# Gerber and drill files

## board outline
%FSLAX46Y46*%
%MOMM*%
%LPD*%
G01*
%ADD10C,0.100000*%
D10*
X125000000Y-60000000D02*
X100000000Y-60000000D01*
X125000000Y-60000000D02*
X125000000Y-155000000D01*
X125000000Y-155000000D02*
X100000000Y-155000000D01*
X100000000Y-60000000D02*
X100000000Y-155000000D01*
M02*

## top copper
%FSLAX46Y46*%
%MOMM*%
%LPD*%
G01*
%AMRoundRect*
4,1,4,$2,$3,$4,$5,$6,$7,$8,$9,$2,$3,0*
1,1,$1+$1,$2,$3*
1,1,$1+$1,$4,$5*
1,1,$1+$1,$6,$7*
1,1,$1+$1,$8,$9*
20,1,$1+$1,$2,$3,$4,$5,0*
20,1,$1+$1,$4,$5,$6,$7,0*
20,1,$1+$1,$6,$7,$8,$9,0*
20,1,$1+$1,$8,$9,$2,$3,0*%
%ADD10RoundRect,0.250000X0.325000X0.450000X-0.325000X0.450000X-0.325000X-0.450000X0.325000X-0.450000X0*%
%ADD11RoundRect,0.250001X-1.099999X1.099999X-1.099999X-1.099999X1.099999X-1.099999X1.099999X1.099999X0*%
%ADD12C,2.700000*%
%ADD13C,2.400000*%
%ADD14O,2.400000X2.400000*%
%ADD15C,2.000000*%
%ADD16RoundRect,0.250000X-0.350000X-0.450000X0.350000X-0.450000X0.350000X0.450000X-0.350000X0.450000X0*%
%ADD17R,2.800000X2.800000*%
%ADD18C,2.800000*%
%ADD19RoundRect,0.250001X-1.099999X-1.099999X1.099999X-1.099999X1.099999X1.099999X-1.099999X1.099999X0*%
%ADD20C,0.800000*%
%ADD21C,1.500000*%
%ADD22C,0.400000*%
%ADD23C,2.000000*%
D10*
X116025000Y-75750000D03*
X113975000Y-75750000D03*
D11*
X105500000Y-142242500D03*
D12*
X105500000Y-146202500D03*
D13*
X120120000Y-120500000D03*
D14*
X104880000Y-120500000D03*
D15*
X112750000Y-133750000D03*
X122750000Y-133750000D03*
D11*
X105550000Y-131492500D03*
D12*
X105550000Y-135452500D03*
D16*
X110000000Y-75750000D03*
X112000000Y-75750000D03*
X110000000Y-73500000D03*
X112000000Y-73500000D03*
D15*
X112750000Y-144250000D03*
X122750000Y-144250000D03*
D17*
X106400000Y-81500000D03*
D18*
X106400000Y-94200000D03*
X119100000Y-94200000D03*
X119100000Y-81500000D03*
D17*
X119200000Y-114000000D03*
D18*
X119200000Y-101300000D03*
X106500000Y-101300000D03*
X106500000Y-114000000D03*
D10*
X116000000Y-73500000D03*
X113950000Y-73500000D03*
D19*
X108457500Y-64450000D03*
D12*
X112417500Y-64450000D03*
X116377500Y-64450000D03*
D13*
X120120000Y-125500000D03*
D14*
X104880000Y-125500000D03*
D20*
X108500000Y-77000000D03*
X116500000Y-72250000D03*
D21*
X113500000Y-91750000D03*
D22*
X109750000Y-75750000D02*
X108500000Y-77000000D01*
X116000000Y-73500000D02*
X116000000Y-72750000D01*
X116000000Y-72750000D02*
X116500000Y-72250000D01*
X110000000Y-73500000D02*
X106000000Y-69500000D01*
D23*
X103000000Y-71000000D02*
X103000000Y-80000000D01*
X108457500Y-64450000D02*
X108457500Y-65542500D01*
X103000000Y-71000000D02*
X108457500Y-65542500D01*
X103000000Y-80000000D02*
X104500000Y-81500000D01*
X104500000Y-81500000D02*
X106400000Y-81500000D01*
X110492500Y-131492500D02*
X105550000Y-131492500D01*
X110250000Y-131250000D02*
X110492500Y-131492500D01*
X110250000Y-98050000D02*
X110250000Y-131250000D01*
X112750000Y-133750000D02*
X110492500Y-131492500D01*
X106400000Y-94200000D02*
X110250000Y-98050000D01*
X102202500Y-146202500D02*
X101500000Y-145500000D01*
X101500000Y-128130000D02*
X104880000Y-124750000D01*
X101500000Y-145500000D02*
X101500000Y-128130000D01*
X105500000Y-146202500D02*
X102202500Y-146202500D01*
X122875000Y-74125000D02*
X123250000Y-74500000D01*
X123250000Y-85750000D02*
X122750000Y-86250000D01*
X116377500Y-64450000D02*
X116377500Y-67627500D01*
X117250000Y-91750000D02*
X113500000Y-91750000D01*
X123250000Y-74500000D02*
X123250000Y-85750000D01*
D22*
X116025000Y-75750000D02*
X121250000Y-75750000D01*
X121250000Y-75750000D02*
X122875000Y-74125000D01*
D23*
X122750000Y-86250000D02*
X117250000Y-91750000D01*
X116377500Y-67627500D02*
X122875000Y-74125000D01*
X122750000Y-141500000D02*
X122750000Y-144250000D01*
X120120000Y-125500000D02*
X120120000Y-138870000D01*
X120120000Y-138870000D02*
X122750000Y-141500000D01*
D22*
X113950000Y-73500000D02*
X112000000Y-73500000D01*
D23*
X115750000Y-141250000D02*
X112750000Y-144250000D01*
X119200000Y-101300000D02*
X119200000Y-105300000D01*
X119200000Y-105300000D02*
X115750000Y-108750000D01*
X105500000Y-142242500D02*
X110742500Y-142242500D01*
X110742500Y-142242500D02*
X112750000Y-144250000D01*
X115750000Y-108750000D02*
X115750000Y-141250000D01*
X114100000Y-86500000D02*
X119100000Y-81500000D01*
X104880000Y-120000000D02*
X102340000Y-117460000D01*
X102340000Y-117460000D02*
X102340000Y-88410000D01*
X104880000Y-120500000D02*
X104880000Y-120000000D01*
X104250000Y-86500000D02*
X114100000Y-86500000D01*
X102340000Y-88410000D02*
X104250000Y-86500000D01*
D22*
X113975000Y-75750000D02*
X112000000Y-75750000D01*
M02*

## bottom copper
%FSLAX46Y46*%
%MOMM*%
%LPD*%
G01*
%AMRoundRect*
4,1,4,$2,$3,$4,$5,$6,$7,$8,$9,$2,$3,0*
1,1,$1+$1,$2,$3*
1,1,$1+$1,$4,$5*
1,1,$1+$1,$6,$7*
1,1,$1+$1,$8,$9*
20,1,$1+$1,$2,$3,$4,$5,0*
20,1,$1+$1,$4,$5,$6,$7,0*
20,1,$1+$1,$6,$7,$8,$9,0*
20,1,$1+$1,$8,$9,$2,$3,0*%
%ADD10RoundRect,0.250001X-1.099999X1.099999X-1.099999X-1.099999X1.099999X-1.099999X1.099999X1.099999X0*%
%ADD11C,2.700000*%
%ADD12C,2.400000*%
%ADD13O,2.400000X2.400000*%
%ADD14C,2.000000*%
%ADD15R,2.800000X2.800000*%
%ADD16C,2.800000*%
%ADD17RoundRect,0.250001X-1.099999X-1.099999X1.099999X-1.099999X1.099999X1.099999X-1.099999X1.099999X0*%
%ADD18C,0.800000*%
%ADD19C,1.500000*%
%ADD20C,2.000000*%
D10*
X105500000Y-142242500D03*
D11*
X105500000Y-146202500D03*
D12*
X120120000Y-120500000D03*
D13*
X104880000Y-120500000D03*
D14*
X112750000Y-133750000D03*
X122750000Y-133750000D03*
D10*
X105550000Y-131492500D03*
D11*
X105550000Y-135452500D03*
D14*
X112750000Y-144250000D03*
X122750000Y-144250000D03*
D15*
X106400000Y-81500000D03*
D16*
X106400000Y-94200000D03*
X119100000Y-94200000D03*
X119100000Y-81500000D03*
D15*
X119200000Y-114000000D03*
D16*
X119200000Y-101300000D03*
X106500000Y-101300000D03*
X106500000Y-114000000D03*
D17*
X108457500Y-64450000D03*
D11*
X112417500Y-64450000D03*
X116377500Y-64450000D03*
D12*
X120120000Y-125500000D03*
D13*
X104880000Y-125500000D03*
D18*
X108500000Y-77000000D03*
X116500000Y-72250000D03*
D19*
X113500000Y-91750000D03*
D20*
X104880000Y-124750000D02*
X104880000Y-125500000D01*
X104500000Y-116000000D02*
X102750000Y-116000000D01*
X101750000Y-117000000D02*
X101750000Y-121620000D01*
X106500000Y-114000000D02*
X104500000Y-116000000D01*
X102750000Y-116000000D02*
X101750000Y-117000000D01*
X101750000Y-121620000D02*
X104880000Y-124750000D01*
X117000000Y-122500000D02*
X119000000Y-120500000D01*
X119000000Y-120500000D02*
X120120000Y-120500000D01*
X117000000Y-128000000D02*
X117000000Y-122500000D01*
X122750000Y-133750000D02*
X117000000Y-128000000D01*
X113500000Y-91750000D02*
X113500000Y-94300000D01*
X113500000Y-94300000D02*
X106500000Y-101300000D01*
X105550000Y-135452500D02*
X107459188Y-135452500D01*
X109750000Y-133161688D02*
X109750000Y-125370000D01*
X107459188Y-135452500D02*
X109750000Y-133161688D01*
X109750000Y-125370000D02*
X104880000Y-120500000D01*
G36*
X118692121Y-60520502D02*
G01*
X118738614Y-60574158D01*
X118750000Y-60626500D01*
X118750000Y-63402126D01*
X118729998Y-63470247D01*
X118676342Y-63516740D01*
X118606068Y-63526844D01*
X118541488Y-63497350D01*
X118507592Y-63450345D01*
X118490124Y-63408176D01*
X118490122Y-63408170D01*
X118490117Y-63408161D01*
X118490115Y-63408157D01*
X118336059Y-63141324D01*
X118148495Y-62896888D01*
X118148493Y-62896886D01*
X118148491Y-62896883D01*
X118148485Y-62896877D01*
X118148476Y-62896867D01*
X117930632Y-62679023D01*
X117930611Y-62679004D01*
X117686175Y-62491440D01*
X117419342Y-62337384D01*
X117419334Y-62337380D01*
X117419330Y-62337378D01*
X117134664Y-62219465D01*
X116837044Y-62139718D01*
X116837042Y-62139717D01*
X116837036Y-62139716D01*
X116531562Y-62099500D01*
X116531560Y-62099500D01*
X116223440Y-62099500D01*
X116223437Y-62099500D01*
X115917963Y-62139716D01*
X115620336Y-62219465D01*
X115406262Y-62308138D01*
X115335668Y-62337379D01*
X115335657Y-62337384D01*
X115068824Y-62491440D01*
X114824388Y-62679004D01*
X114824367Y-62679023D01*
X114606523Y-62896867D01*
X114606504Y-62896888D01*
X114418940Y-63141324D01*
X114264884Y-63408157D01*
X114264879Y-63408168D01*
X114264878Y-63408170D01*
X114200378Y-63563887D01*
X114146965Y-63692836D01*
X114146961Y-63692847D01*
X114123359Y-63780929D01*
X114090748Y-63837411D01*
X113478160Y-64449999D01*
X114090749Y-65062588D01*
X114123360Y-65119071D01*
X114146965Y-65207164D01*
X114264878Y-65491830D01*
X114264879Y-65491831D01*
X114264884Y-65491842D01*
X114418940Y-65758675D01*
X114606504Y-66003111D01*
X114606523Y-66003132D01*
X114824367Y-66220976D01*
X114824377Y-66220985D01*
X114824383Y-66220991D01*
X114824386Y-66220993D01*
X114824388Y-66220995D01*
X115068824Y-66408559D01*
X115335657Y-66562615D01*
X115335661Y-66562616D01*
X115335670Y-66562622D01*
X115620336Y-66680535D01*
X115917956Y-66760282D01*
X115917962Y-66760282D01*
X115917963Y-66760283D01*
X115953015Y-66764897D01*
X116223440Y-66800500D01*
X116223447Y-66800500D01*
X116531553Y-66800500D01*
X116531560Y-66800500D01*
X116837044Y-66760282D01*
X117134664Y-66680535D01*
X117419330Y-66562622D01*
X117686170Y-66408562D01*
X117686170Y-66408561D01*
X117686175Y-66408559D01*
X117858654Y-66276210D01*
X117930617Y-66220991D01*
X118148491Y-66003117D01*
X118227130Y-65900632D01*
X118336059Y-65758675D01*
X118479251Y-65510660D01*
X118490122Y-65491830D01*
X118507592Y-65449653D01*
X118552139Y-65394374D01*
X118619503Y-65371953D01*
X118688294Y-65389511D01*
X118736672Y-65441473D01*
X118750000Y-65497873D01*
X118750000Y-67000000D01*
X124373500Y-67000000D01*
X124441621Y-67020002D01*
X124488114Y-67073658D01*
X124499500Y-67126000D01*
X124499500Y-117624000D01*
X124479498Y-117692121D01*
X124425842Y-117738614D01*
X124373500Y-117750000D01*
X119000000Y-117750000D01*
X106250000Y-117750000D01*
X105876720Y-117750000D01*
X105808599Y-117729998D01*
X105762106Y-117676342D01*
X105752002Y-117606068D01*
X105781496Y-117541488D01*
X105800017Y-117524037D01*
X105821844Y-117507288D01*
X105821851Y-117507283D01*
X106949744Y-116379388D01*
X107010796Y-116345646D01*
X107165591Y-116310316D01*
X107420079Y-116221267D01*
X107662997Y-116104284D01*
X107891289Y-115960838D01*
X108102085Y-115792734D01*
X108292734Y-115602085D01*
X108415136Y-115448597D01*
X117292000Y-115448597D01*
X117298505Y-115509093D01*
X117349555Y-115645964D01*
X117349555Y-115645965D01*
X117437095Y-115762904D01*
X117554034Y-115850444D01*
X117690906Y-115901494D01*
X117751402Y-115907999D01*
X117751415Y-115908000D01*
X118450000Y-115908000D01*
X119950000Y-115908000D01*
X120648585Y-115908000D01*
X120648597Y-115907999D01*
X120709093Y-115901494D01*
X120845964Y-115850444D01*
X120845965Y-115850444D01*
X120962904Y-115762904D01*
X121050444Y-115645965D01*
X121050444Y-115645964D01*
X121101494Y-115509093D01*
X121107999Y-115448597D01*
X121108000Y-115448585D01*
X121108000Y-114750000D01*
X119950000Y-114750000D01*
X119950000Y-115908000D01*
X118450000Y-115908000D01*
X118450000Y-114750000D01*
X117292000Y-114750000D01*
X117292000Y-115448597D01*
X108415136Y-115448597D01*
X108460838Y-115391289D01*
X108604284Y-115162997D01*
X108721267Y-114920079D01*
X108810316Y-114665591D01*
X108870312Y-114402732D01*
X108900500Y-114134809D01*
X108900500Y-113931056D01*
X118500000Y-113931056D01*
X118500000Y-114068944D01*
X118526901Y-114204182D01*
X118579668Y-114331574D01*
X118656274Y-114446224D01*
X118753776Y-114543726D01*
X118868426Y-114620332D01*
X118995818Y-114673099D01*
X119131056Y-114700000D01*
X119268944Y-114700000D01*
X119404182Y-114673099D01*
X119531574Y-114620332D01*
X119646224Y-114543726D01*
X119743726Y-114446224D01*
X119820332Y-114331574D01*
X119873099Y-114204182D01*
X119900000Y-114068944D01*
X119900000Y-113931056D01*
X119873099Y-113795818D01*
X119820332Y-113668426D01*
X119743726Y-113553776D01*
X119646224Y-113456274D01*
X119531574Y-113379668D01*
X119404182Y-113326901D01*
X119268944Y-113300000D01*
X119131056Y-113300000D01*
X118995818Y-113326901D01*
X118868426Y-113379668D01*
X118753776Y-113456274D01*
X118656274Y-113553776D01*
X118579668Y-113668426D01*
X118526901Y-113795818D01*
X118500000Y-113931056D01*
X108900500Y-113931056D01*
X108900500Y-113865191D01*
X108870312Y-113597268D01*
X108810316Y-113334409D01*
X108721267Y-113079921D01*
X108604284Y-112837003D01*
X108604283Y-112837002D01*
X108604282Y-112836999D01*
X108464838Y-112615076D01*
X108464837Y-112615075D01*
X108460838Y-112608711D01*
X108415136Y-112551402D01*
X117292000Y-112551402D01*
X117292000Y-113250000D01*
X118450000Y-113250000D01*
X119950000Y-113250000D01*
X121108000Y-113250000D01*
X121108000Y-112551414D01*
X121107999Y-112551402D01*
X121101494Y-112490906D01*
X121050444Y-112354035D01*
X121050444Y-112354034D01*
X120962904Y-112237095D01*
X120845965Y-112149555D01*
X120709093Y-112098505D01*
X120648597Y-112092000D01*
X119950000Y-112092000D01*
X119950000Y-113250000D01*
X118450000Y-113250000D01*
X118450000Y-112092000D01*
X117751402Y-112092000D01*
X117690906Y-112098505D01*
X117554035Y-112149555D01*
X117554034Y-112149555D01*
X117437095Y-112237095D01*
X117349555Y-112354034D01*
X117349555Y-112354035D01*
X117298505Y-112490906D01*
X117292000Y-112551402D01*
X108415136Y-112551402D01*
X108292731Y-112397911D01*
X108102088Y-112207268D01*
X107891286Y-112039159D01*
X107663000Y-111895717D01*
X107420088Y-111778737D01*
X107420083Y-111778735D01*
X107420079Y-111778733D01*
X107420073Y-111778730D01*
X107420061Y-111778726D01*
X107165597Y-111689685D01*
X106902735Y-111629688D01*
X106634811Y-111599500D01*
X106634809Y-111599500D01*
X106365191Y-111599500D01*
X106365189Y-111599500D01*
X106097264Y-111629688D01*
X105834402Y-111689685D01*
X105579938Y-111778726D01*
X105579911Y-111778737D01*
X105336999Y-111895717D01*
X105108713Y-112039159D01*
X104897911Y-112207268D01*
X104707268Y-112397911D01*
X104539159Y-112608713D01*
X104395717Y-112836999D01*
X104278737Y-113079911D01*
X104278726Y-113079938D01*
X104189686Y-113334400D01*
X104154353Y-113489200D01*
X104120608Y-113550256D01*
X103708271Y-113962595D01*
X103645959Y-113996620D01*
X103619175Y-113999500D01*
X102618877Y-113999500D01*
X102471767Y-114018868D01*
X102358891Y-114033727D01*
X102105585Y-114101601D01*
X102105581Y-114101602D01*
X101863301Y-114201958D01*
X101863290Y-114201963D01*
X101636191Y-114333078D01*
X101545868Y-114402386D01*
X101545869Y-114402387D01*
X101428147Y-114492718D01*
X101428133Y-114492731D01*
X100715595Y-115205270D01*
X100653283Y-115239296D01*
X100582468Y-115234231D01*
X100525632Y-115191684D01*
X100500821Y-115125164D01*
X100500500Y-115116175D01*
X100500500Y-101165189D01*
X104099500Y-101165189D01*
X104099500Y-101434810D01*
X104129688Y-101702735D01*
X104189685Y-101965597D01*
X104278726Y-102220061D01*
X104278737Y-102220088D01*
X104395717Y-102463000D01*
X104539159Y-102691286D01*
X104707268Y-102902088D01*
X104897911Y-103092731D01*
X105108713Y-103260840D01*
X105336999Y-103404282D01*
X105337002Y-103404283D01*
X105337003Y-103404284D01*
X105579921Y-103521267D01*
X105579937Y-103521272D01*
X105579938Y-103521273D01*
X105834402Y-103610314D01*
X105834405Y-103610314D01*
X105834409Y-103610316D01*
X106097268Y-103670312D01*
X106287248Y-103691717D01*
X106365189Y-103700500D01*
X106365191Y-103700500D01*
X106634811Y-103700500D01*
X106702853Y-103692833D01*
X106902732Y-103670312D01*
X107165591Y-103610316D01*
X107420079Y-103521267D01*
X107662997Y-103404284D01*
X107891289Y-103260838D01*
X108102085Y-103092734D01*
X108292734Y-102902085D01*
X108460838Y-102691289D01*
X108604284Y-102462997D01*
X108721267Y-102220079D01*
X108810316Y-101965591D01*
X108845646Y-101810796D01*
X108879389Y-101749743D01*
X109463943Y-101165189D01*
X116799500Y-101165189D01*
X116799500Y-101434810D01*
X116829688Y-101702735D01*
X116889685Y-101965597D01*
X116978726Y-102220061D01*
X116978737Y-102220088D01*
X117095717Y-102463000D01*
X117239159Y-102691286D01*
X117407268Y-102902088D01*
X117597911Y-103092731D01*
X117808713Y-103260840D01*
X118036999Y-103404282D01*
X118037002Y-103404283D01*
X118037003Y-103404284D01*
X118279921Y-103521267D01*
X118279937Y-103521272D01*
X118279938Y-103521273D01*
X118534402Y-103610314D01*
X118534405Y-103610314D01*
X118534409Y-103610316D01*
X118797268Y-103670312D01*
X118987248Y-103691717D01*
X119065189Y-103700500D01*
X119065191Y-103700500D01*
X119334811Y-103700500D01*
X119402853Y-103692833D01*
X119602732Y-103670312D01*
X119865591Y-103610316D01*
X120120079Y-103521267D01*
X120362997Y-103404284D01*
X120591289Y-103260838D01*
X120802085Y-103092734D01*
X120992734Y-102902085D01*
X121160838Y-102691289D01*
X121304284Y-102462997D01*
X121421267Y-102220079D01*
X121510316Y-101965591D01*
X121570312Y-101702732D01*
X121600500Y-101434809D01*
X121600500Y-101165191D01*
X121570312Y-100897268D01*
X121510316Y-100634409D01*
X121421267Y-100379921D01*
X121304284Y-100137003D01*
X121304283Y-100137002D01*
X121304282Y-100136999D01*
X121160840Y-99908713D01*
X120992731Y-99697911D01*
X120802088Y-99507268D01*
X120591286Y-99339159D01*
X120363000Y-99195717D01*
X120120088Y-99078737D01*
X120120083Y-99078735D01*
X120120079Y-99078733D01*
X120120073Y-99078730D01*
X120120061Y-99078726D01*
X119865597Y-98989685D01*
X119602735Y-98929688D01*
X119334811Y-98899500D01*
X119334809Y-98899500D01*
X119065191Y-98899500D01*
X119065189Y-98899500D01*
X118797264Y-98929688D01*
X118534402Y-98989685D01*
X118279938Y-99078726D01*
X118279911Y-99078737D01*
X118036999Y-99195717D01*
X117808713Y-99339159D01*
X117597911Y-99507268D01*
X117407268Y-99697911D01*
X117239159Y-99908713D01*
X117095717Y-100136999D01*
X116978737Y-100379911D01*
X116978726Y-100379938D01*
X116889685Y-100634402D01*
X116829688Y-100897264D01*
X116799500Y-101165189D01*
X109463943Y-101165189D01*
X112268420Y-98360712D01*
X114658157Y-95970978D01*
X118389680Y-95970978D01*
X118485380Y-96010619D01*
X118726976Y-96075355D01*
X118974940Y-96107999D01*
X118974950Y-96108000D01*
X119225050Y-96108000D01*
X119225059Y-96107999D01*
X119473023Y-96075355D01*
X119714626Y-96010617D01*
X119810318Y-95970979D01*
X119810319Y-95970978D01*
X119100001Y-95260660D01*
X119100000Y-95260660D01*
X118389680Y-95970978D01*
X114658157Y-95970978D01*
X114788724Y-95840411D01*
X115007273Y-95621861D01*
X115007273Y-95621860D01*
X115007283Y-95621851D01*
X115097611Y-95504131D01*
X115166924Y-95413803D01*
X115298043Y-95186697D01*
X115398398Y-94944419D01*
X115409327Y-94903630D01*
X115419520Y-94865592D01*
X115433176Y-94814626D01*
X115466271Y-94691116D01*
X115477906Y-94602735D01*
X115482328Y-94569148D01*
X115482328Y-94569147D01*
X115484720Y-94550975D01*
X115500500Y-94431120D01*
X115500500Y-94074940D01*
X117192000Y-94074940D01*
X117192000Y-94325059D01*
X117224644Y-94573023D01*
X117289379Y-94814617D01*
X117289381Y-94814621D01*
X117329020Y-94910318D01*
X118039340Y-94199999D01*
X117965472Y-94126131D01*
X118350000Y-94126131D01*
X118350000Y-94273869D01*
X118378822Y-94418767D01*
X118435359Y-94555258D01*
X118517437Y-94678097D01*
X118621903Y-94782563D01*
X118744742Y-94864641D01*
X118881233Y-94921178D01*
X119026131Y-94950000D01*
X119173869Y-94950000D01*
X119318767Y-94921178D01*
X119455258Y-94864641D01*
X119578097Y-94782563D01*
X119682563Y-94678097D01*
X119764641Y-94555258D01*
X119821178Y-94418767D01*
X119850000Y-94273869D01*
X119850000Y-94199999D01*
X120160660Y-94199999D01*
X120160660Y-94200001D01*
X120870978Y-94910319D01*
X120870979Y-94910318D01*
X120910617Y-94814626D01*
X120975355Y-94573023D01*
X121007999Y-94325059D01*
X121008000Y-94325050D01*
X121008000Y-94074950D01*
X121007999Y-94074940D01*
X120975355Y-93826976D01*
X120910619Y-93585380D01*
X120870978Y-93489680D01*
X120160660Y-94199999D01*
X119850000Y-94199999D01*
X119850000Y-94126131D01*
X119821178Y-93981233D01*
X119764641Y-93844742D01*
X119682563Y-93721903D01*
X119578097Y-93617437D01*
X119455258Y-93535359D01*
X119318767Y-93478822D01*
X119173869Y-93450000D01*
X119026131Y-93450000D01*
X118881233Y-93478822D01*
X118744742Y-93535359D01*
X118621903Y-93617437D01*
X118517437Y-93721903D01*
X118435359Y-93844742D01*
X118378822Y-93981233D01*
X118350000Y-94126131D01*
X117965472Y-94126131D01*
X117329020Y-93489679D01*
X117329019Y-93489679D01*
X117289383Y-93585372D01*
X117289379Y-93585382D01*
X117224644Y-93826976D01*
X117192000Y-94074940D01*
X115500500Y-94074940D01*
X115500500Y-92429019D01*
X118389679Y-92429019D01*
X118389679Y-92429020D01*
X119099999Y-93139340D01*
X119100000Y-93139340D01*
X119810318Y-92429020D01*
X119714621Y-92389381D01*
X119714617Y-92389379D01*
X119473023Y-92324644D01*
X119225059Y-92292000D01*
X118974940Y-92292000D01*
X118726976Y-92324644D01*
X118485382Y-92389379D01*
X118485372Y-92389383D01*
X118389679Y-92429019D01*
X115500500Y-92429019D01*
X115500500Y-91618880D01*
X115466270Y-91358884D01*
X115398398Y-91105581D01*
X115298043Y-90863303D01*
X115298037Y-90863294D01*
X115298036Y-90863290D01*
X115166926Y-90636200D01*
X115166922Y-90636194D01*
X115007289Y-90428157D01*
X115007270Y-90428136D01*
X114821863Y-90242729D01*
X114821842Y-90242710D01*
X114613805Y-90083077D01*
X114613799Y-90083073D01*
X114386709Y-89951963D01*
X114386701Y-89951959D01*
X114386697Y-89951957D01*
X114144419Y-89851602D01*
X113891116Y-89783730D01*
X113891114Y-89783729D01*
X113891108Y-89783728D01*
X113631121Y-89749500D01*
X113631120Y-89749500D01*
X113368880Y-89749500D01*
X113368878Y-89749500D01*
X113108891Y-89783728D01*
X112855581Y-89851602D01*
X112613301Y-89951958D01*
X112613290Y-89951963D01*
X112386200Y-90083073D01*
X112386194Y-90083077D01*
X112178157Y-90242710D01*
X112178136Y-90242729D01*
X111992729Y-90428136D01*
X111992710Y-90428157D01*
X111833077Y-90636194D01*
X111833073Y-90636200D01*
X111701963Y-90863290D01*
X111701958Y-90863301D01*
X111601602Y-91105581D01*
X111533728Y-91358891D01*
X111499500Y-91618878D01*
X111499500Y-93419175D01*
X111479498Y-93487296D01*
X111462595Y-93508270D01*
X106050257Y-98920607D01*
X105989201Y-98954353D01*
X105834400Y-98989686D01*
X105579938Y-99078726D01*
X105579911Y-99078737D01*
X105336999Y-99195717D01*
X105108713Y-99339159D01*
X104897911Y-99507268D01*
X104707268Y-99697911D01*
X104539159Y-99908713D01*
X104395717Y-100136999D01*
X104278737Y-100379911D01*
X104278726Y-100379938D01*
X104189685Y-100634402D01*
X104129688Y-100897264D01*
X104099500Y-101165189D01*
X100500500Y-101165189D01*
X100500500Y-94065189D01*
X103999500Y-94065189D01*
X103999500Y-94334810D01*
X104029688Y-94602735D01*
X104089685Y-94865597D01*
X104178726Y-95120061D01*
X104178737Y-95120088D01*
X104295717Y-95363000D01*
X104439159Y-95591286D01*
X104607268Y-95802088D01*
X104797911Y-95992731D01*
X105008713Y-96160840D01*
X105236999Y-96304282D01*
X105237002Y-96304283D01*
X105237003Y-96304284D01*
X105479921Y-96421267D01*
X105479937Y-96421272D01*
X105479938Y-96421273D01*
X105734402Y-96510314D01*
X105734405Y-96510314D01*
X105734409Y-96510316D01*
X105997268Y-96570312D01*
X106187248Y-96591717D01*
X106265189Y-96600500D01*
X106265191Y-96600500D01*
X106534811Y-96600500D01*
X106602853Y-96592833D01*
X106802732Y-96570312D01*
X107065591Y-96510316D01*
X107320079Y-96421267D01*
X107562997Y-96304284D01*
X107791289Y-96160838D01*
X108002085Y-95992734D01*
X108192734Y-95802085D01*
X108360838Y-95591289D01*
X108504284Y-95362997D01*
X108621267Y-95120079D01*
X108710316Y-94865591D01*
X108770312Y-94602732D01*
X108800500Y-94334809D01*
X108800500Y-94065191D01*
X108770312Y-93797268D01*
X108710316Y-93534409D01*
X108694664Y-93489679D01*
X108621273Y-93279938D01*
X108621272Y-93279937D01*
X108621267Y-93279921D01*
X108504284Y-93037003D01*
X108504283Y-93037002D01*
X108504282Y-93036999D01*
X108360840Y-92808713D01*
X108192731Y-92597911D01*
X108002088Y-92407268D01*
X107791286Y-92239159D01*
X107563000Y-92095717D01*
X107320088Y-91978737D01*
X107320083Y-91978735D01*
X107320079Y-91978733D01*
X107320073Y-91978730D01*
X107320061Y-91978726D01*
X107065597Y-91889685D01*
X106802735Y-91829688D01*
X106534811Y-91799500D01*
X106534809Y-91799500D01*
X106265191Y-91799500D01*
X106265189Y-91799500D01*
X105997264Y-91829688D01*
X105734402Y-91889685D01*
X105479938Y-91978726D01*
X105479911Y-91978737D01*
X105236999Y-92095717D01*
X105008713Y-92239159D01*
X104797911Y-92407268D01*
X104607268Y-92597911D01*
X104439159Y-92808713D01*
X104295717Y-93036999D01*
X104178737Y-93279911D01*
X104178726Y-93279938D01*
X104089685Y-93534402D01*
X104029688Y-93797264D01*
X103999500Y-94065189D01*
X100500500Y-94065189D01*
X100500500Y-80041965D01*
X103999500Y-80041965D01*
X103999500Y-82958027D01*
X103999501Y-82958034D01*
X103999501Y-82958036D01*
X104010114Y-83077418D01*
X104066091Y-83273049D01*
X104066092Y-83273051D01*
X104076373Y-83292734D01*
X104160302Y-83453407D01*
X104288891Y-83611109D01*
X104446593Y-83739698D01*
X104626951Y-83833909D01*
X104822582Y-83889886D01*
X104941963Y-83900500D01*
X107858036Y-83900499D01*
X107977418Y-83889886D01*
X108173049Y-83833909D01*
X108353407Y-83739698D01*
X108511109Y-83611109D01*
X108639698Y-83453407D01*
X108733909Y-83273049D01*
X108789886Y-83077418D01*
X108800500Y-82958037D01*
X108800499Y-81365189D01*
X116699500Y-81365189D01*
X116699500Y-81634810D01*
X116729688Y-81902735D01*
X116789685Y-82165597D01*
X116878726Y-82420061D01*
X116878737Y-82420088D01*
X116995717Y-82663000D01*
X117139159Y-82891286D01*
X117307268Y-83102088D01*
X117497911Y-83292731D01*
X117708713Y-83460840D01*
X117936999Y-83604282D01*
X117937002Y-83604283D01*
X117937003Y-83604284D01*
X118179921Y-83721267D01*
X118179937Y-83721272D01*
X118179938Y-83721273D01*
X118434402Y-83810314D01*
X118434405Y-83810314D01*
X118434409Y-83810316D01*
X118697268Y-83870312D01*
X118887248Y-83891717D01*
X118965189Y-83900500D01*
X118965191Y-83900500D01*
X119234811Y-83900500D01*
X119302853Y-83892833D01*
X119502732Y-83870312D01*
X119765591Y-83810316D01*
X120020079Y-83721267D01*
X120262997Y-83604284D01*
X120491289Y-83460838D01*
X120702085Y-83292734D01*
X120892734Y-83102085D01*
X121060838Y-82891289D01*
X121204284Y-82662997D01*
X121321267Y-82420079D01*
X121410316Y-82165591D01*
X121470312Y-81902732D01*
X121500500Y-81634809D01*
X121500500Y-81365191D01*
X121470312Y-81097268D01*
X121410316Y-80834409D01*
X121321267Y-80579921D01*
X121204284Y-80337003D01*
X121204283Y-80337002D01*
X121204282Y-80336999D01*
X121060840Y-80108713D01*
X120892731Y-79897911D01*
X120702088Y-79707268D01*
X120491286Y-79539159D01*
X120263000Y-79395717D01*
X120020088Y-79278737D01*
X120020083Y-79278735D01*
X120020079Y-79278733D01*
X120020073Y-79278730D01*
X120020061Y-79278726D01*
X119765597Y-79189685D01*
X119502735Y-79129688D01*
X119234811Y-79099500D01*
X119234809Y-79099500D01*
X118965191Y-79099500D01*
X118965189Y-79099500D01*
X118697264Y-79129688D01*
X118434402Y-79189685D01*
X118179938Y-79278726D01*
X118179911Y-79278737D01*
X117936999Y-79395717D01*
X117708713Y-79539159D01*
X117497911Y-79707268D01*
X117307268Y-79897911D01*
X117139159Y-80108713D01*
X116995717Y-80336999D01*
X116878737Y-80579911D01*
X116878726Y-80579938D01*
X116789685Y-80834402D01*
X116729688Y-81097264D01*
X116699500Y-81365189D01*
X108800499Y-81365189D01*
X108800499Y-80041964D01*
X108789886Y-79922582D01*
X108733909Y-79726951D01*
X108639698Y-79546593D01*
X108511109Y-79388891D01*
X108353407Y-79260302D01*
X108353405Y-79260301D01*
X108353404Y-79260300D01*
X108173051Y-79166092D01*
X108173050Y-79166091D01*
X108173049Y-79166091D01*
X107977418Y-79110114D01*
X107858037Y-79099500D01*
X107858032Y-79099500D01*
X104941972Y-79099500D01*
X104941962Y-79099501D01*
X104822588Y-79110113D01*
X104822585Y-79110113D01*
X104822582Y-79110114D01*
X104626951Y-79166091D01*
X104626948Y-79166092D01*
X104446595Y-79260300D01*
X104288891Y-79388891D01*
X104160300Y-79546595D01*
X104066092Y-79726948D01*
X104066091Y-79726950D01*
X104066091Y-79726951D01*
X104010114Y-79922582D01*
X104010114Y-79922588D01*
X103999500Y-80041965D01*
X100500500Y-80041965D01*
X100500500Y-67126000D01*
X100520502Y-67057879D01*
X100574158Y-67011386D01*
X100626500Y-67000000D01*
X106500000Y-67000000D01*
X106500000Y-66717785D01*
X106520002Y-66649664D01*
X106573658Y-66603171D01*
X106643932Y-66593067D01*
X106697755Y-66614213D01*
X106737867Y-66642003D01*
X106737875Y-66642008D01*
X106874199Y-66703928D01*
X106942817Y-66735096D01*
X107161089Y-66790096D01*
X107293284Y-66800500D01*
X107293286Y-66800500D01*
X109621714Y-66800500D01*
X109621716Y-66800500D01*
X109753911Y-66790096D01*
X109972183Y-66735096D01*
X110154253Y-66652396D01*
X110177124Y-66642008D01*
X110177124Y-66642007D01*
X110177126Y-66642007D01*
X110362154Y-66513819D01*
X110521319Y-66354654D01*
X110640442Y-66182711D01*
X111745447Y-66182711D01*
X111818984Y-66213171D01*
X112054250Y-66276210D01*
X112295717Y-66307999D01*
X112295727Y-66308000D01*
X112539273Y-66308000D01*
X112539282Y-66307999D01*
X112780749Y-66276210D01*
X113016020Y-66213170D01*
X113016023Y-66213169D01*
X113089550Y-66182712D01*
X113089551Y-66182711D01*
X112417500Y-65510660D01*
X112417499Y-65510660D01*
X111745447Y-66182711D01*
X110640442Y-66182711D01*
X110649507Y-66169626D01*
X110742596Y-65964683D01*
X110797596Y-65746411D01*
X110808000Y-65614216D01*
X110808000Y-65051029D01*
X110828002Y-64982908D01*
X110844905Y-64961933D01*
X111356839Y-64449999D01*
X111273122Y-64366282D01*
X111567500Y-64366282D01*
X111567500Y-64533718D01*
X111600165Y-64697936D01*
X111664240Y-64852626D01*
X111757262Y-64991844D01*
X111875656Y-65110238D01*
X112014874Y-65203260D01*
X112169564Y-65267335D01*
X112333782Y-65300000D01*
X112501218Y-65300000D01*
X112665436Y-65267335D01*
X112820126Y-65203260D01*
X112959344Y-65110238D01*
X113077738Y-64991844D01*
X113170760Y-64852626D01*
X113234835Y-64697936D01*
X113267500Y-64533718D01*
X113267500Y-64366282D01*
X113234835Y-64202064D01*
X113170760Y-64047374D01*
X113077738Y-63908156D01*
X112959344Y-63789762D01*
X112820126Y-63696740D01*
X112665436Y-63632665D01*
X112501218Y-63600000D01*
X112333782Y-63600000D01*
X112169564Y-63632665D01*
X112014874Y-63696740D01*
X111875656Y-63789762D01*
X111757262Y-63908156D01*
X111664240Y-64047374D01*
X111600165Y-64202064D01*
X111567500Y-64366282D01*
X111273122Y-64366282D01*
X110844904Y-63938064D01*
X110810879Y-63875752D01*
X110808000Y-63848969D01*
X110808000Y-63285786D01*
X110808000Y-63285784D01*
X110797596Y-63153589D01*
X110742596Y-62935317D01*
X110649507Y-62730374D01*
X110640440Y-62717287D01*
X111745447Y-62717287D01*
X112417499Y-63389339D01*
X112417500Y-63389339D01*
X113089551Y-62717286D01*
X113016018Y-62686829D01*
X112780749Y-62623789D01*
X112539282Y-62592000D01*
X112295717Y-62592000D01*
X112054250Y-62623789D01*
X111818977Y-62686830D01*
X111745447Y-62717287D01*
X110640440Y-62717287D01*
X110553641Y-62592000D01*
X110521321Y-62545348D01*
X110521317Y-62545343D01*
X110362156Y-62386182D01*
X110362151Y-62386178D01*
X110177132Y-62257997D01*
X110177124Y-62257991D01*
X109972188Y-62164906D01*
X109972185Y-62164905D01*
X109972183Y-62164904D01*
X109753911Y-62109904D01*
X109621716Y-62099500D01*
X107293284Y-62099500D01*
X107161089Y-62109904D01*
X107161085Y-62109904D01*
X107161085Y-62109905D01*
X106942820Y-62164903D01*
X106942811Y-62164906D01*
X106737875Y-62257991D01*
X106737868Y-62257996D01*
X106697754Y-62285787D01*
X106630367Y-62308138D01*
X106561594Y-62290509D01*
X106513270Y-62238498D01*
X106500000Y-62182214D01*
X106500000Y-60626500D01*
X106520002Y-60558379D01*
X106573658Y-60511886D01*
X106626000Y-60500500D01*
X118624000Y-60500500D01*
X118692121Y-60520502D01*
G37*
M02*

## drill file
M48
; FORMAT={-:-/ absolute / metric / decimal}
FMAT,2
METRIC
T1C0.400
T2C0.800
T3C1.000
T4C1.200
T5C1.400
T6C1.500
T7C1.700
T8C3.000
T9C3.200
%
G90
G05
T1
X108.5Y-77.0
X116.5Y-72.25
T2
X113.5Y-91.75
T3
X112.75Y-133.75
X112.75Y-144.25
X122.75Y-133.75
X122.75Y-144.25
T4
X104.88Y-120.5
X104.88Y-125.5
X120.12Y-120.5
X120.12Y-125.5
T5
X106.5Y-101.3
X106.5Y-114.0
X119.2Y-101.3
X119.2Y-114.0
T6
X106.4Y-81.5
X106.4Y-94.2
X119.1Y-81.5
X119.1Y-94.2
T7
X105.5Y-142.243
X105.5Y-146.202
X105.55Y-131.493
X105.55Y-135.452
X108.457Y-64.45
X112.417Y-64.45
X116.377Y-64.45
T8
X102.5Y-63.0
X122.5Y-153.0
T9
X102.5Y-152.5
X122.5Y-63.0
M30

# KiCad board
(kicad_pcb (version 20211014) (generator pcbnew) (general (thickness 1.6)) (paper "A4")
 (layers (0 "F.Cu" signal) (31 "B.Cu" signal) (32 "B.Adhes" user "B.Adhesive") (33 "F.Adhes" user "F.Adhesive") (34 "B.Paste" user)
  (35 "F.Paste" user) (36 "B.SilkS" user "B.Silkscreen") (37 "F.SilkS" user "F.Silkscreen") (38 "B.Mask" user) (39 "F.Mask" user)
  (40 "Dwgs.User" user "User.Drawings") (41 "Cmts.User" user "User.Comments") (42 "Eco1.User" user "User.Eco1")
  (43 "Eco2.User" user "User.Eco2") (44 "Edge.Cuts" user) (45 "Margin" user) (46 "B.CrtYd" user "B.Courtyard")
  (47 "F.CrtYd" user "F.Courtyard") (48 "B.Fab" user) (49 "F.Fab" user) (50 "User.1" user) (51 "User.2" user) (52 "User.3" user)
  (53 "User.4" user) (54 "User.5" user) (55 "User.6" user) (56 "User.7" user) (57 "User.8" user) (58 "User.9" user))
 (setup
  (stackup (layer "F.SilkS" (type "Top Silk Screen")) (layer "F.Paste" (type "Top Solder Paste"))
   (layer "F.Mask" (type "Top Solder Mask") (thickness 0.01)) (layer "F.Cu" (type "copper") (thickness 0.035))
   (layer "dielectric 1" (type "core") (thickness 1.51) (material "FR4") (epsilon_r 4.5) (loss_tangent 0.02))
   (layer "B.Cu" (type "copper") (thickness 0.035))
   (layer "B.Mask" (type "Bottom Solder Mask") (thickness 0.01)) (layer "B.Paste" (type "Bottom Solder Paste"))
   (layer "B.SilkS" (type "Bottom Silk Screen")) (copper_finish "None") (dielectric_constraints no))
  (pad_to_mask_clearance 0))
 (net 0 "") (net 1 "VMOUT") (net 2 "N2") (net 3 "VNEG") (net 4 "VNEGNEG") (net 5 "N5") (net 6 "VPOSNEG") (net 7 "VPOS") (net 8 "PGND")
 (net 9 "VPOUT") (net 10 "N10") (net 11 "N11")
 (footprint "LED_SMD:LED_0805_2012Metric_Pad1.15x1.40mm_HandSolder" (layer "F.Cu") (at 115 75.75 180)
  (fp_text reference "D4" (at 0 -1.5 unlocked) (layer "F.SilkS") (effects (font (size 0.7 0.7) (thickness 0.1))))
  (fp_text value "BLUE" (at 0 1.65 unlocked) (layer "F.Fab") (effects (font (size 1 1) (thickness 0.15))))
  (pad "1" smd roundrect (at -1.025 0 180) (size 1.15 1.4) (layers "F.Cu" "F.Paste" "F.Mask") (roundrect_rratio 0.2173913043)
   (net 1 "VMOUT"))
  (pad "2" smd roundrect (at 1.025 0 180) (size 1.15 1.4) (layers "F.Cu" "F.Paste" "F.Mask") (roundrect_rratio 0.2173913043) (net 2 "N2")))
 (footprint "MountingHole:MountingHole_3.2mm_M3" (layer "F.Cu") (at 122.5 63)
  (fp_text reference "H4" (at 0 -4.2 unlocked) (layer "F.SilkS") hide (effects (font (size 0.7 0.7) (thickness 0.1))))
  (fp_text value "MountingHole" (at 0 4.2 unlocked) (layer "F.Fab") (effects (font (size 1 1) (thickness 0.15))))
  (pad "" np_thru_hole circle (at 0 0) (size 3.2 3.2) (drill 3.2) (layers *.Cu *.Mask)))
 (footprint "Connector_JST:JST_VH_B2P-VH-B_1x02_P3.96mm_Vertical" (layer "F.Cu") (at 105.5 142.2425 -90)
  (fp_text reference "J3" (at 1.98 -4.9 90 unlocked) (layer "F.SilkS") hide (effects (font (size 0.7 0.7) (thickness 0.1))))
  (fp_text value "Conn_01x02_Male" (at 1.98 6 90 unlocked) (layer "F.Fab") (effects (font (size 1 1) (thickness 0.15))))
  (pad "1" thru_hole roundrect (at 0 0 270) (size 2.7 2.7) (drill 1.7) (layers *.Cu *.Mask) (roundrect_rratio 0.09259296296) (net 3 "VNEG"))
  (pad "2" thru_hole circle (at 3.96 0 270) (size 2.7 2.7) (drill 1.7) (layers *.Cu *.Mask) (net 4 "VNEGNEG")))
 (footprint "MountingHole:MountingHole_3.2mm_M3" (layer "F.Cu") (at 102.5 152.5)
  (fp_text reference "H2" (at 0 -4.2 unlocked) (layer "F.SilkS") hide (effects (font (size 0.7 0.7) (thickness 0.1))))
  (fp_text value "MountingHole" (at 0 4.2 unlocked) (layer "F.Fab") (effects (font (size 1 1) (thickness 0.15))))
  (pad "" np_thru_hole circle (at 0 0) (size 3.2 3.2) (drill 3.2) (layers *.Cu *.Mask)))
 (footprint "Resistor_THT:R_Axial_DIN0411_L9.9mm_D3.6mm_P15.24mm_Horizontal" (layer "F.Cu") (at 120.12 120.5 180)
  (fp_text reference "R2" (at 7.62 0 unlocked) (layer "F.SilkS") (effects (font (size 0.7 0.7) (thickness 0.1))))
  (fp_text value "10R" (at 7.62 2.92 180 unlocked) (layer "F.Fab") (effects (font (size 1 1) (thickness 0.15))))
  (pad "1" thru_hole circle (at 0 0 180) (size 2.4 2.4) (drill 1.2) (layers *.Cu *.Mask) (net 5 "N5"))
  (pad "2" thru_hole oval (at 15.24 0 180) (size 2.4 2.4) (drill 1.2) (layers *.Cu *.Mask) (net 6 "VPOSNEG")))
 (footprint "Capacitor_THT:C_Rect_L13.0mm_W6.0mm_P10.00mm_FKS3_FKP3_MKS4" (layer "F.Cu") (at 112.75 133.75)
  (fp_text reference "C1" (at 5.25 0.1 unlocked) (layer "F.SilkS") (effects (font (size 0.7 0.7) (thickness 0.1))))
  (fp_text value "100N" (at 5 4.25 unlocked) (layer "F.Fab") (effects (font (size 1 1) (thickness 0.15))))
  (pad "1" thru_hole circle (at 0 0) (size 2 2) (drill 1) (layers *.Cu *.Mask) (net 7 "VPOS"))
  (pad "2" thru_hole circle (at 10 0) (size 2 2) (drill 1) (layers *.Cu *.Mask) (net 5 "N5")))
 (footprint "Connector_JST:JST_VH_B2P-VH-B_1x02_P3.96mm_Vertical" (layer "F.Cu") (at 105.55 131.4925 -90)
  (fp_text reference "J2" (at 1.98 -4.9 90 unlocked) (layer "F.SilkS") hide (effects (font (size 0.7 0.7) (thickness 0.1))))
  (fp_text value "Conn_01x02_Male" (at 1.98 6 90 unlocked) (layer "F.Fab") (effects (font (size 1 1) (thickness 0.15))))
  (pad "1" thru_hole roundrect (at 0 0 270) (size 2.7 2.7) (drill 1.7) (layers *.Cu *.Mask) (roundrect_rratio 0.09259296296) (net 7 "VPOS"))
  (pad "2" thru_hole circle (at 3.96 0 270) (size 2.7 2.7) (drill 1.7) (layers *.Cu *.Mask) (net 6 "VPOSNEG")))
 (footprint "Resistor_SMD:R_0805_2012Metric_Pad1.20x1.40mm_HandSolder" (layer "F.Cu") (at 111 75.75)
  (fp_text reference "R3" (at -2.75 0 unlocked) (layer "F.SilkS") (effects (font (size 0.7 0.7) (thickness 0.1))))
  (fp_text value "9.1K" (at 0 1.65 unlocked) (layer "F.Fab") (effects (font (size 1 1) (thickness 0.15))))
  (pad "1" smd roundrect (at -1 0) (size 1.2 1.4) (layers "F.Cu" "F.Paste" "F.Mask") (roundrect_rratio 0.2083333333) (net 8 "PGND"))
  (pad "2" smd roundrect (at 1 0) (size 1.2 1.4) (layers "F.Cu" "F.Paste" "F.Mask") (roundrect_rratio 0.2083333333) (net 2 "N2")))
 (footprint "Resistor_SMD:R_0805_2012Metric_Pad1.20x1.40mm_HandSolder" (layer "F.Cu") (at 111 73.5)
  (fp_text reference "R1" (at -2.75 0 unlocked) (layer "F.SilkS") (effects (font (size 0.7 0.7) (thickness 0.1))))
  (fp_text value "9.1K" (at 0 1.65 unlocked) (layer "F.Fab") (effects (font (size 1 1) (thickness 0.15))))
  (pad "1" smd roundrect (at -1 0) (size 1.2 1.4) (layers "F.Cu" "F.Paste" "F.Mask") (roundrect_rratio 0.2083333333) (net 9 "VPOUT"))
  (pad "2" smd roundrect (at 1 0) (size 1.2 1.4) (layers "F.Cu" "F.Paste" "F.Mask") (roundrect_rratio 0.2083333333) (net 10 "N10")))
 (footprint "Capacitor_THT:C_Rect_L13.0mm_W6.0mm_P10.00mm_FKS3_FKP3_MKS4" (layer "F.Cu") (at 112.75 144.25)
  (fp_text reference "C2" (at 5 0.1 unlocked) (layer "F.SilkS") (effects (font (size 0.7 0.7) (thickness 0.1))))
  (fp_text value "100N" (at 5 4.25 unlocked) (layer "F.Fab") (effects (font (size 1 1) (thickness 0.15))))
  (pad "1" thru_hole circle (at 0 0) (size 2 2) (drill 1) (layers *.Cu *.Mask) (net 3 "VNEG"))
  (pad "2" thru_hole circle (at 10 0) (size 2 2) (drill 1) (layers *.Cu *.Mask) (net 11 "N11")))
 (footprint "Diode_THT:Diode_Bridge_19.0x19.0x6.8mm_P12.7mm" (layer "F.Cu") (at 106.4 81.5)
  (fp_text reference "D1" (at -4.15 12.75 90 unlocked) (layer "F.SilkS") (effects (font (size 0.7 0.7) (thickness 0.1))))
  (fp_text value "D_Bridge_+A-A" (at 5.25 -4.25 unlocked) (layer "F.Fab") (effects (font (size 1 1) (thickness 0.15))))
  (pad "1" thru_hole rect (at 0 0 180) (size 2.8 2.8) (drill 1.5) (layers *.Cu *.Mask) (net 9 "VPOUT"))
  (pad "2" thru_hole circle (at 0 12.7 180) (size 2.8 2.8) (drill 1.5) (layers *.Cu *.Mask) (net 7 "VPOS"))
  (pad "3" thru_hole circle (at 12.7 12.7 180) (size 2.8 2.8) (drill 1.5) (layers *.Cu *.Mask) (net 8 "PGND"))
  (pad "4" thru_hole circle (at 12.7 0 180) (size 2.8 2.8) (drill 1.5) (layers *.Cu *.Mask) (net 6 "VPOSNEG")))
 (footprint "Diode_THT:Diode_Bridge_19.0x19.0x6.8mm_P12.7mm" (layer "F.Cu") (at 119.2 114 180)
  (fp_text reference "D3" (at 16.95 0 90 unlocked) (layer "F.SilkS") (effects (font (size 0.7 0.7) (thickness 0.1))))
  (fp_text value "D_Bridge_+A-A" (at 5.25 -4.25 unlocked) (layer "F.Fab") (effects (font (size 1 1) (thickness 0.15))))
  (pad "1" thru_hole rect (at 0 0) (size 2.8 2.8) (drill 1.4) (layers *.Cu *.Mask) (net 8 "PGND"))
  (pad "2" thru_hole circle (at 0 12.7) (size 2.8 2.8) (drill 1.4) (layers *.Cu *.Mask) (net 3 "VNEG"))
  (pad "3" thru_hole circle (at 12.7 12.7) (size 2.8 2.8) (drill 1.4) (layers *.Cu *.Mask) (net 1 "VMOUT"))
  (pad "4" thru_hole circle (at 12.7 0) (size 2.8 2.8) (drill 1.4) (layers *.Cu *.Mask) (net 4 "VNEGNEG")))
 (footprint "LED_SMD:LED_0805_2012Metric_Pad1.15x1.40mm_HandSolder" (layer "F.Cu") (at 114.975 73.5 180)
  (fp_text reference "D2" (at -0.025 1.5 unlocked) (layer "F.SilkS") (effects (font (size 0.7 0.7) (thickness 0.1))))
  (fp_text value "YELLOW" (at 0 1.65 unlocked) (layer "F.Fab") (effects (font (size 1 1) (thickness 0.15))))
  (pad "1" smd roundrect (at -1.025 0 180) (size 1.15 1.4) (layers "F.Cu" "F.Paste" "F.Mask") (roundrect_rratio 0.2173913043) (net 8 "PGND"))
  (pad "2" smd roundrect (at 1.025 0 180) (size 1.15 1.4) (layers "F.Cu" "F.Paste" "F.Mask") (roundrect_rratio 0.2173913043) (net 10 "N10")))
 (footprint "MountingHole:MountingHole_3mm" (layer "F.Cu") (at 122.5 153)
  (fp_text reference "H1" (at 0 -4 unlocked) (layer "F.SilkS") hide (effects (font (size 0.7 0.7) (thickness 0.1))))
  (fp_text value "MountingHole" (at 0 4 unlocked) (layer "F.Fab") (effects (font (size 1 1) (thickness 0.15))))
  (pad "" np_thru_hole circle (at 0 0) (size 3 3) (drill 3) (layers *.Cu *.Mask)))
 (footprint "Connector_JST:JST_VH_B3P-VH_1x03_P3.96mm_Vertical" (layer "F.Cu") (at 108.4575 64.45)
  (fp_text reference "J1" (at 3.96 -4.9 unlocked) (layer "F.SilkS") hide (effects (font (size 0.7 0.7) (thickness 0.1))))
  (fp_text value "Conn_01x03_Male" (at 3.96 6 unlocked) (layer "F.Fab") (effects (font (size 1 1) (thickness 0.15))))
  (pad "1" thru_hole roundrect (at 0 0) (size 2.7 2.7) (drill 1.7) (layers *.Cu *.Mask) (roundrect_rratio 0.09259296296) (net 9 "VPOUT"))
  (pad "2" thru_hole circle (at 3.96 0) (size 2.7 2.7) (drill 1.7) (layers *.Cu *.Mask) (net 8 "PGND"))
  (pad "3" thru_hole circle (at 7.92 0) (size 2.7 2.7) (drill 1.7) (layers *.Cu *.Mask) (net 1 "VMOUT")))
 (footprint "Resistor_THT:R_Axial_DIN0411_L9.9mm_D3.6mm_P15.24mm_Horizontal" (layer "F.Cu") (at 120.12 125.5 180)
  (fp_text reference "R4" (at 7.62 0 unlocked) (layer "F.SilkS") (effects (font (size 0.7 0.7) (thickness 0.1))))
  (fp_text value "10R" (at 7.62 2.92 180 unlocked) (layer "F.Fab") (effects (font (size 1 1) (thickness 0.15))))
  (pad "1" thru_hole circle (at 0 0 180) (size 2.4 2.4) (drill 1.2) (layers *.Cu *.Mask) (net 11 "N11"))
  (pad "2" thru_hole oval (at 15.24 0 180) (size 2.4 2.4) (drill 1.2) (layers *.Cu *.Mask) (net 4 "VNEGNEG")))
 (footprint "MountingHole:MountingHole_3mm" (layer "F.Cu") (at 102.5 63)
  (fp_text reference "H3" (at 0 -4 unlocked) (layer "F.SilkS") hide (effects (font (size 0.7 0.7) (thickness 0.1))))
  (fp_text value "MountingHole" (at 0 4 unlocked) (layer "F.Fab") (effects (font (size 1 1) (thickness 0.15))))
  (pad "" np_thru_hole circle (at 0 0) (size 3 3) (drill 3) (layers *.Cu *.Mask)))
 (gr_line (start 125 60) (end 100 60) (layer "Edge.Cuts") (width 0.1))
 (gr_line (start 125 60) (end 125 155) (layer "Edge.Cuts") (width 0.1))
 (gr_line (start 125 155) (end 100 155) (layer "Edge.Cuts") (width 0.1))
 (gr_line (start 100 60) (end 100 155) (layer "Edge.Cuts") (width 0.1))
 (segment (start 109.75 75.75) (end 108.5 77) (width 0.4) (layer "F.Cu") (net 8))
 (segment (start 116 73.5) (end 116 72.75) (width 0.4) (layer "F.Cu") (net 8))
 (segment (start 116 72.75) (end 116.5 72.25) (width 0.4) (layer "F.Cu") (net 8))
 (via (at 108.5 77) (size 0.8) (drill 0.4) (layers "F.Cu" "B.Cu") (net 8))
 (via (at 116.5 72.25) (size 0.8) (drill 0.4) (layers "F.Cu" "B.Cu") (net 8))
 (segment (start 110 73.5) (end 106 69.5) (width 0.4) (layer "F.Cu") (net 9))
 (segment (start 103 71) (end 103 80) (width 2) (layer "F.Cu") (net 9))
 (segment (start 108.4575 64.45) (end 108.4575 65.5425) (width 2) (layer "F.Cu") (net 9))
 (segment (start 103 71) (end 108.4575 65.5425) (width 2) (layer "F.Cu") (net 9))
 (segment (start 103 80) (end 104.5 81.5) (width 2) (layer "F.Cu") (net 9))
 (segment (start 104.5 81.5) (end 106.4 81.5) (width 2) (layer "F.Cu") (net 9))
 (segment (start 110.4925 131.4925) (end 105.55 131.4925) (width 2) (layer "F.Cu") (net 7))
 (segment (start 110.25 131.25) (end 110.4925 131.4925) (width 2) (layer "F.Cu") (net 7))
 (segment (start 110.25 98.05) (end 110.25 131.25) (width 2) (layer "F.Cu") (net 7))
 (segment (start 112.75 133.75) (end 110.4925 131.4925) (width 2) (layer "F.Cu") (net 7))
 (segment (start 106.4 94.2) (end 110.25 98.05) (width 2) (layer "F.Cu") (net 7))
 (segment (start 102.2025 146.2025) (end 101.5 145.5) (width 2) (layer "F.Cu") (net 4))
 (segment (start 101.5 128.13) (end 104.88 124.75) (width 2) (layer "F.Cu") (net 4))
 (segment (start 101.5 145.5) (end 101.5 128.13) (width 2) (layer "F.Cu") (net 4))
 (segment (start 105.5 146.2025) (end 102.2025 146.2025) (width 2) (layer "F.Cu") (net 4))
 (segment (start 104.88 124.75) (end 104.88 125.5) (width 2) (layer "B.Cu") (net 4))
 (segment (start 104.5 116) (end 102.75 116) (width 2) (layer "B.Cu") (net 4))
 (segment (start 101.75 117) (end 101.75 121.62) (width 2) (layer "B.Cu") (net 4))
 (segment (start 106.5 114) (end 104.5 116) (width 2) (layer "B.Cu") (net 4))
 (segment (start 102.75 116) (end 101.75 117) (width 2) (layer "B.Cu") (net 4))
 (segment (start 101.75 121.62) (end 104.88 124.75) (width 2) (layer "B.Cu") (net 4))
 (segment (start 117 122.5) (end 119 120.5) (width 2) (layer "B.Cu") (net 5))
 (segment (start 119 120.5) (end 120.12 120.5) (width 2) (layer "B.Cu") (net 5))
 (segment (start 117 128) (end 117 122.5) (width 2) (layer "B.Cu") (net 5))
 (segment (start 122.75 133.75) (end 117 128) (width 2) (layer "B.Cu") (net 5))
 (segment (start 122.875 74.125) (end 123.25 74.5) (width 2) (layer "F.Cu") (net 1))
 (segment (start 123.25 85.75) (end 122.75 86.25) (width 2) (layer "F.Cu") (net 1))
 (segment (start 116.3775 64.45) (end 116.3775 67.6275) (width 2) (layer "F.Cu") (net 1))
 (segment (start 117.25 91.75) (end 113.5 91.75) (width 2) (layer "F.Cu") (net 1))
 (segment (start 123.25 74.5) (end 123.25 85.75) (width 2) (layer "F.Cu") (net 1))
 (segment (start 116.025 75.75) (end 121.25 75.75) (width 0.4) (layer "F.Cu") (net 1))
 (segment (start 121.25 75.75) (end 122.875 74.125) (width 0.4) (layer "F.Cu") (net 1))
 (segment (start 122.75 86.25) (end 117.25 91.75) (width 2) (layer "F.Cu") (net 1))
 (segment (start 116.3775 67.6275) (end 122.875 74.125) (width 2) (layer "F.Cu") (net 1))
 (via (at 113.5 91.75) (size 1.5) (drill 0.8) (layers "F.Cu" "B.Cu") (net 1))
 (segment (start 113.5 91.75) (end 113.5 94.3) (width 2) (layer "B.Cu") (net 1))
 (segment (start 113.5 94.3) (end 106.5 101.3) (width 2) (layer "B.Cu") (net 1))
 (segment (start 122.75 141.5) (end 122.75 144.25) (width 2) (layer "F.Cu") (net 11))
 (segment (start 120.12 125.5) (end 120.12 138.87) (width 2) (layer "F.Cu") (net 11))
 (segment (start 120.12 138.87) (end 122.75 141.5) (width 2) (layer "F.Cu") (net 11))
 (segment (start 113.95 73.5) (end 112 73.5) (width 0.4) (layer "F.Cu") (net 10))
 (segment (start 115.75 141.25) (end 112.75 144.25) (width 2) (layer "F.Cu") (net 3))
 (segment (start 119.2 101.3) (end 119.2 105.3) (width 2) (layer "F.Cu") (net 3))
 (segment (start 119.2 105.3) (end 115.75 108.75) (width 2) (layer "F.Cu") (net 3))
 (segment (start 105.5 142.2425) (end 110.7425 142.2425) (width 2) (layer "F.Cu") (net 3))
 (segment (start 110.7425 142.2425) (end 112.75 144.25) (width 2) (layer "F.Cu") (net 3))
 (segment (start 115.75 108.75) (end 115.75 141.25) (width 2) (layer "F.Cu") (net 3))
 (segment (start 114.1 86.5) (end 119.1 81.5) (width 2) (layer "F.Cu") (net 6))
 (segment (start 104.88 120) (end 102.34 117.46) (width 2) (layer "F.Cu") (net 6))
 (segment (start 102.34 117.46) (end 102.34 88.41) (width 2) (layer "F.Cu") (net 6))
 (segment (start 104.88 120.5) (end 104.88 120) (width 2) (layer "F.Cu") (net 6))
 (segment (start 104.25 86.5) (end 114.1 86.5) (width 2) (layer "F.Cu") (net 6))
 (segment (start 102.34 88.41) (end 104.25 86.5) (width 2) (layer "F.Cu") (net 6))
 (segment (start 105.55 135.4525) (end 107.459188 135.4525) (width 2) (layer "B.Cu") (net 6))
 (segment (start 109.75 133.161688) (end 109.75 125.37) (width 2) (layer "B.Cu") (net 6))
 (segment (start 107.459188 135.4525) (end 109.75 133.161688) (width 2) (layer "B.Cu") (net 6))
 (segment (start 109.75 125.37) (end 104.88 120.5) (width 2) (layer "B.Cu") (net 6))
 (segment (start 113.975 75.75) (end 112 75.75) (width 0.4) (layer "F.Cu") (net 2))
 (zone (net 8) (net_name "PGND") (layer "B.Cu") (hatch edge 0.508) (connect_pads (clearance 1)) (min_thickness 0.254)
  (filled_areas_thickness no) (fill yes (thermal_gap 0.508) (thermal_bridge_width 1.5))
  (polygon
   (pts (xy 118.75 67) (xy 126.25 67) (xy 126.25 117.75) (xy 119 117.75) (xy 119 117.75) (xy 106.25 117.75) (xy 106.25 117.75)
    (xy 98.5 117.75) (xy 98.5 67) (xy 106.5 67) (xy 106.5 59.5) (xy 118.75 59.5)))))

